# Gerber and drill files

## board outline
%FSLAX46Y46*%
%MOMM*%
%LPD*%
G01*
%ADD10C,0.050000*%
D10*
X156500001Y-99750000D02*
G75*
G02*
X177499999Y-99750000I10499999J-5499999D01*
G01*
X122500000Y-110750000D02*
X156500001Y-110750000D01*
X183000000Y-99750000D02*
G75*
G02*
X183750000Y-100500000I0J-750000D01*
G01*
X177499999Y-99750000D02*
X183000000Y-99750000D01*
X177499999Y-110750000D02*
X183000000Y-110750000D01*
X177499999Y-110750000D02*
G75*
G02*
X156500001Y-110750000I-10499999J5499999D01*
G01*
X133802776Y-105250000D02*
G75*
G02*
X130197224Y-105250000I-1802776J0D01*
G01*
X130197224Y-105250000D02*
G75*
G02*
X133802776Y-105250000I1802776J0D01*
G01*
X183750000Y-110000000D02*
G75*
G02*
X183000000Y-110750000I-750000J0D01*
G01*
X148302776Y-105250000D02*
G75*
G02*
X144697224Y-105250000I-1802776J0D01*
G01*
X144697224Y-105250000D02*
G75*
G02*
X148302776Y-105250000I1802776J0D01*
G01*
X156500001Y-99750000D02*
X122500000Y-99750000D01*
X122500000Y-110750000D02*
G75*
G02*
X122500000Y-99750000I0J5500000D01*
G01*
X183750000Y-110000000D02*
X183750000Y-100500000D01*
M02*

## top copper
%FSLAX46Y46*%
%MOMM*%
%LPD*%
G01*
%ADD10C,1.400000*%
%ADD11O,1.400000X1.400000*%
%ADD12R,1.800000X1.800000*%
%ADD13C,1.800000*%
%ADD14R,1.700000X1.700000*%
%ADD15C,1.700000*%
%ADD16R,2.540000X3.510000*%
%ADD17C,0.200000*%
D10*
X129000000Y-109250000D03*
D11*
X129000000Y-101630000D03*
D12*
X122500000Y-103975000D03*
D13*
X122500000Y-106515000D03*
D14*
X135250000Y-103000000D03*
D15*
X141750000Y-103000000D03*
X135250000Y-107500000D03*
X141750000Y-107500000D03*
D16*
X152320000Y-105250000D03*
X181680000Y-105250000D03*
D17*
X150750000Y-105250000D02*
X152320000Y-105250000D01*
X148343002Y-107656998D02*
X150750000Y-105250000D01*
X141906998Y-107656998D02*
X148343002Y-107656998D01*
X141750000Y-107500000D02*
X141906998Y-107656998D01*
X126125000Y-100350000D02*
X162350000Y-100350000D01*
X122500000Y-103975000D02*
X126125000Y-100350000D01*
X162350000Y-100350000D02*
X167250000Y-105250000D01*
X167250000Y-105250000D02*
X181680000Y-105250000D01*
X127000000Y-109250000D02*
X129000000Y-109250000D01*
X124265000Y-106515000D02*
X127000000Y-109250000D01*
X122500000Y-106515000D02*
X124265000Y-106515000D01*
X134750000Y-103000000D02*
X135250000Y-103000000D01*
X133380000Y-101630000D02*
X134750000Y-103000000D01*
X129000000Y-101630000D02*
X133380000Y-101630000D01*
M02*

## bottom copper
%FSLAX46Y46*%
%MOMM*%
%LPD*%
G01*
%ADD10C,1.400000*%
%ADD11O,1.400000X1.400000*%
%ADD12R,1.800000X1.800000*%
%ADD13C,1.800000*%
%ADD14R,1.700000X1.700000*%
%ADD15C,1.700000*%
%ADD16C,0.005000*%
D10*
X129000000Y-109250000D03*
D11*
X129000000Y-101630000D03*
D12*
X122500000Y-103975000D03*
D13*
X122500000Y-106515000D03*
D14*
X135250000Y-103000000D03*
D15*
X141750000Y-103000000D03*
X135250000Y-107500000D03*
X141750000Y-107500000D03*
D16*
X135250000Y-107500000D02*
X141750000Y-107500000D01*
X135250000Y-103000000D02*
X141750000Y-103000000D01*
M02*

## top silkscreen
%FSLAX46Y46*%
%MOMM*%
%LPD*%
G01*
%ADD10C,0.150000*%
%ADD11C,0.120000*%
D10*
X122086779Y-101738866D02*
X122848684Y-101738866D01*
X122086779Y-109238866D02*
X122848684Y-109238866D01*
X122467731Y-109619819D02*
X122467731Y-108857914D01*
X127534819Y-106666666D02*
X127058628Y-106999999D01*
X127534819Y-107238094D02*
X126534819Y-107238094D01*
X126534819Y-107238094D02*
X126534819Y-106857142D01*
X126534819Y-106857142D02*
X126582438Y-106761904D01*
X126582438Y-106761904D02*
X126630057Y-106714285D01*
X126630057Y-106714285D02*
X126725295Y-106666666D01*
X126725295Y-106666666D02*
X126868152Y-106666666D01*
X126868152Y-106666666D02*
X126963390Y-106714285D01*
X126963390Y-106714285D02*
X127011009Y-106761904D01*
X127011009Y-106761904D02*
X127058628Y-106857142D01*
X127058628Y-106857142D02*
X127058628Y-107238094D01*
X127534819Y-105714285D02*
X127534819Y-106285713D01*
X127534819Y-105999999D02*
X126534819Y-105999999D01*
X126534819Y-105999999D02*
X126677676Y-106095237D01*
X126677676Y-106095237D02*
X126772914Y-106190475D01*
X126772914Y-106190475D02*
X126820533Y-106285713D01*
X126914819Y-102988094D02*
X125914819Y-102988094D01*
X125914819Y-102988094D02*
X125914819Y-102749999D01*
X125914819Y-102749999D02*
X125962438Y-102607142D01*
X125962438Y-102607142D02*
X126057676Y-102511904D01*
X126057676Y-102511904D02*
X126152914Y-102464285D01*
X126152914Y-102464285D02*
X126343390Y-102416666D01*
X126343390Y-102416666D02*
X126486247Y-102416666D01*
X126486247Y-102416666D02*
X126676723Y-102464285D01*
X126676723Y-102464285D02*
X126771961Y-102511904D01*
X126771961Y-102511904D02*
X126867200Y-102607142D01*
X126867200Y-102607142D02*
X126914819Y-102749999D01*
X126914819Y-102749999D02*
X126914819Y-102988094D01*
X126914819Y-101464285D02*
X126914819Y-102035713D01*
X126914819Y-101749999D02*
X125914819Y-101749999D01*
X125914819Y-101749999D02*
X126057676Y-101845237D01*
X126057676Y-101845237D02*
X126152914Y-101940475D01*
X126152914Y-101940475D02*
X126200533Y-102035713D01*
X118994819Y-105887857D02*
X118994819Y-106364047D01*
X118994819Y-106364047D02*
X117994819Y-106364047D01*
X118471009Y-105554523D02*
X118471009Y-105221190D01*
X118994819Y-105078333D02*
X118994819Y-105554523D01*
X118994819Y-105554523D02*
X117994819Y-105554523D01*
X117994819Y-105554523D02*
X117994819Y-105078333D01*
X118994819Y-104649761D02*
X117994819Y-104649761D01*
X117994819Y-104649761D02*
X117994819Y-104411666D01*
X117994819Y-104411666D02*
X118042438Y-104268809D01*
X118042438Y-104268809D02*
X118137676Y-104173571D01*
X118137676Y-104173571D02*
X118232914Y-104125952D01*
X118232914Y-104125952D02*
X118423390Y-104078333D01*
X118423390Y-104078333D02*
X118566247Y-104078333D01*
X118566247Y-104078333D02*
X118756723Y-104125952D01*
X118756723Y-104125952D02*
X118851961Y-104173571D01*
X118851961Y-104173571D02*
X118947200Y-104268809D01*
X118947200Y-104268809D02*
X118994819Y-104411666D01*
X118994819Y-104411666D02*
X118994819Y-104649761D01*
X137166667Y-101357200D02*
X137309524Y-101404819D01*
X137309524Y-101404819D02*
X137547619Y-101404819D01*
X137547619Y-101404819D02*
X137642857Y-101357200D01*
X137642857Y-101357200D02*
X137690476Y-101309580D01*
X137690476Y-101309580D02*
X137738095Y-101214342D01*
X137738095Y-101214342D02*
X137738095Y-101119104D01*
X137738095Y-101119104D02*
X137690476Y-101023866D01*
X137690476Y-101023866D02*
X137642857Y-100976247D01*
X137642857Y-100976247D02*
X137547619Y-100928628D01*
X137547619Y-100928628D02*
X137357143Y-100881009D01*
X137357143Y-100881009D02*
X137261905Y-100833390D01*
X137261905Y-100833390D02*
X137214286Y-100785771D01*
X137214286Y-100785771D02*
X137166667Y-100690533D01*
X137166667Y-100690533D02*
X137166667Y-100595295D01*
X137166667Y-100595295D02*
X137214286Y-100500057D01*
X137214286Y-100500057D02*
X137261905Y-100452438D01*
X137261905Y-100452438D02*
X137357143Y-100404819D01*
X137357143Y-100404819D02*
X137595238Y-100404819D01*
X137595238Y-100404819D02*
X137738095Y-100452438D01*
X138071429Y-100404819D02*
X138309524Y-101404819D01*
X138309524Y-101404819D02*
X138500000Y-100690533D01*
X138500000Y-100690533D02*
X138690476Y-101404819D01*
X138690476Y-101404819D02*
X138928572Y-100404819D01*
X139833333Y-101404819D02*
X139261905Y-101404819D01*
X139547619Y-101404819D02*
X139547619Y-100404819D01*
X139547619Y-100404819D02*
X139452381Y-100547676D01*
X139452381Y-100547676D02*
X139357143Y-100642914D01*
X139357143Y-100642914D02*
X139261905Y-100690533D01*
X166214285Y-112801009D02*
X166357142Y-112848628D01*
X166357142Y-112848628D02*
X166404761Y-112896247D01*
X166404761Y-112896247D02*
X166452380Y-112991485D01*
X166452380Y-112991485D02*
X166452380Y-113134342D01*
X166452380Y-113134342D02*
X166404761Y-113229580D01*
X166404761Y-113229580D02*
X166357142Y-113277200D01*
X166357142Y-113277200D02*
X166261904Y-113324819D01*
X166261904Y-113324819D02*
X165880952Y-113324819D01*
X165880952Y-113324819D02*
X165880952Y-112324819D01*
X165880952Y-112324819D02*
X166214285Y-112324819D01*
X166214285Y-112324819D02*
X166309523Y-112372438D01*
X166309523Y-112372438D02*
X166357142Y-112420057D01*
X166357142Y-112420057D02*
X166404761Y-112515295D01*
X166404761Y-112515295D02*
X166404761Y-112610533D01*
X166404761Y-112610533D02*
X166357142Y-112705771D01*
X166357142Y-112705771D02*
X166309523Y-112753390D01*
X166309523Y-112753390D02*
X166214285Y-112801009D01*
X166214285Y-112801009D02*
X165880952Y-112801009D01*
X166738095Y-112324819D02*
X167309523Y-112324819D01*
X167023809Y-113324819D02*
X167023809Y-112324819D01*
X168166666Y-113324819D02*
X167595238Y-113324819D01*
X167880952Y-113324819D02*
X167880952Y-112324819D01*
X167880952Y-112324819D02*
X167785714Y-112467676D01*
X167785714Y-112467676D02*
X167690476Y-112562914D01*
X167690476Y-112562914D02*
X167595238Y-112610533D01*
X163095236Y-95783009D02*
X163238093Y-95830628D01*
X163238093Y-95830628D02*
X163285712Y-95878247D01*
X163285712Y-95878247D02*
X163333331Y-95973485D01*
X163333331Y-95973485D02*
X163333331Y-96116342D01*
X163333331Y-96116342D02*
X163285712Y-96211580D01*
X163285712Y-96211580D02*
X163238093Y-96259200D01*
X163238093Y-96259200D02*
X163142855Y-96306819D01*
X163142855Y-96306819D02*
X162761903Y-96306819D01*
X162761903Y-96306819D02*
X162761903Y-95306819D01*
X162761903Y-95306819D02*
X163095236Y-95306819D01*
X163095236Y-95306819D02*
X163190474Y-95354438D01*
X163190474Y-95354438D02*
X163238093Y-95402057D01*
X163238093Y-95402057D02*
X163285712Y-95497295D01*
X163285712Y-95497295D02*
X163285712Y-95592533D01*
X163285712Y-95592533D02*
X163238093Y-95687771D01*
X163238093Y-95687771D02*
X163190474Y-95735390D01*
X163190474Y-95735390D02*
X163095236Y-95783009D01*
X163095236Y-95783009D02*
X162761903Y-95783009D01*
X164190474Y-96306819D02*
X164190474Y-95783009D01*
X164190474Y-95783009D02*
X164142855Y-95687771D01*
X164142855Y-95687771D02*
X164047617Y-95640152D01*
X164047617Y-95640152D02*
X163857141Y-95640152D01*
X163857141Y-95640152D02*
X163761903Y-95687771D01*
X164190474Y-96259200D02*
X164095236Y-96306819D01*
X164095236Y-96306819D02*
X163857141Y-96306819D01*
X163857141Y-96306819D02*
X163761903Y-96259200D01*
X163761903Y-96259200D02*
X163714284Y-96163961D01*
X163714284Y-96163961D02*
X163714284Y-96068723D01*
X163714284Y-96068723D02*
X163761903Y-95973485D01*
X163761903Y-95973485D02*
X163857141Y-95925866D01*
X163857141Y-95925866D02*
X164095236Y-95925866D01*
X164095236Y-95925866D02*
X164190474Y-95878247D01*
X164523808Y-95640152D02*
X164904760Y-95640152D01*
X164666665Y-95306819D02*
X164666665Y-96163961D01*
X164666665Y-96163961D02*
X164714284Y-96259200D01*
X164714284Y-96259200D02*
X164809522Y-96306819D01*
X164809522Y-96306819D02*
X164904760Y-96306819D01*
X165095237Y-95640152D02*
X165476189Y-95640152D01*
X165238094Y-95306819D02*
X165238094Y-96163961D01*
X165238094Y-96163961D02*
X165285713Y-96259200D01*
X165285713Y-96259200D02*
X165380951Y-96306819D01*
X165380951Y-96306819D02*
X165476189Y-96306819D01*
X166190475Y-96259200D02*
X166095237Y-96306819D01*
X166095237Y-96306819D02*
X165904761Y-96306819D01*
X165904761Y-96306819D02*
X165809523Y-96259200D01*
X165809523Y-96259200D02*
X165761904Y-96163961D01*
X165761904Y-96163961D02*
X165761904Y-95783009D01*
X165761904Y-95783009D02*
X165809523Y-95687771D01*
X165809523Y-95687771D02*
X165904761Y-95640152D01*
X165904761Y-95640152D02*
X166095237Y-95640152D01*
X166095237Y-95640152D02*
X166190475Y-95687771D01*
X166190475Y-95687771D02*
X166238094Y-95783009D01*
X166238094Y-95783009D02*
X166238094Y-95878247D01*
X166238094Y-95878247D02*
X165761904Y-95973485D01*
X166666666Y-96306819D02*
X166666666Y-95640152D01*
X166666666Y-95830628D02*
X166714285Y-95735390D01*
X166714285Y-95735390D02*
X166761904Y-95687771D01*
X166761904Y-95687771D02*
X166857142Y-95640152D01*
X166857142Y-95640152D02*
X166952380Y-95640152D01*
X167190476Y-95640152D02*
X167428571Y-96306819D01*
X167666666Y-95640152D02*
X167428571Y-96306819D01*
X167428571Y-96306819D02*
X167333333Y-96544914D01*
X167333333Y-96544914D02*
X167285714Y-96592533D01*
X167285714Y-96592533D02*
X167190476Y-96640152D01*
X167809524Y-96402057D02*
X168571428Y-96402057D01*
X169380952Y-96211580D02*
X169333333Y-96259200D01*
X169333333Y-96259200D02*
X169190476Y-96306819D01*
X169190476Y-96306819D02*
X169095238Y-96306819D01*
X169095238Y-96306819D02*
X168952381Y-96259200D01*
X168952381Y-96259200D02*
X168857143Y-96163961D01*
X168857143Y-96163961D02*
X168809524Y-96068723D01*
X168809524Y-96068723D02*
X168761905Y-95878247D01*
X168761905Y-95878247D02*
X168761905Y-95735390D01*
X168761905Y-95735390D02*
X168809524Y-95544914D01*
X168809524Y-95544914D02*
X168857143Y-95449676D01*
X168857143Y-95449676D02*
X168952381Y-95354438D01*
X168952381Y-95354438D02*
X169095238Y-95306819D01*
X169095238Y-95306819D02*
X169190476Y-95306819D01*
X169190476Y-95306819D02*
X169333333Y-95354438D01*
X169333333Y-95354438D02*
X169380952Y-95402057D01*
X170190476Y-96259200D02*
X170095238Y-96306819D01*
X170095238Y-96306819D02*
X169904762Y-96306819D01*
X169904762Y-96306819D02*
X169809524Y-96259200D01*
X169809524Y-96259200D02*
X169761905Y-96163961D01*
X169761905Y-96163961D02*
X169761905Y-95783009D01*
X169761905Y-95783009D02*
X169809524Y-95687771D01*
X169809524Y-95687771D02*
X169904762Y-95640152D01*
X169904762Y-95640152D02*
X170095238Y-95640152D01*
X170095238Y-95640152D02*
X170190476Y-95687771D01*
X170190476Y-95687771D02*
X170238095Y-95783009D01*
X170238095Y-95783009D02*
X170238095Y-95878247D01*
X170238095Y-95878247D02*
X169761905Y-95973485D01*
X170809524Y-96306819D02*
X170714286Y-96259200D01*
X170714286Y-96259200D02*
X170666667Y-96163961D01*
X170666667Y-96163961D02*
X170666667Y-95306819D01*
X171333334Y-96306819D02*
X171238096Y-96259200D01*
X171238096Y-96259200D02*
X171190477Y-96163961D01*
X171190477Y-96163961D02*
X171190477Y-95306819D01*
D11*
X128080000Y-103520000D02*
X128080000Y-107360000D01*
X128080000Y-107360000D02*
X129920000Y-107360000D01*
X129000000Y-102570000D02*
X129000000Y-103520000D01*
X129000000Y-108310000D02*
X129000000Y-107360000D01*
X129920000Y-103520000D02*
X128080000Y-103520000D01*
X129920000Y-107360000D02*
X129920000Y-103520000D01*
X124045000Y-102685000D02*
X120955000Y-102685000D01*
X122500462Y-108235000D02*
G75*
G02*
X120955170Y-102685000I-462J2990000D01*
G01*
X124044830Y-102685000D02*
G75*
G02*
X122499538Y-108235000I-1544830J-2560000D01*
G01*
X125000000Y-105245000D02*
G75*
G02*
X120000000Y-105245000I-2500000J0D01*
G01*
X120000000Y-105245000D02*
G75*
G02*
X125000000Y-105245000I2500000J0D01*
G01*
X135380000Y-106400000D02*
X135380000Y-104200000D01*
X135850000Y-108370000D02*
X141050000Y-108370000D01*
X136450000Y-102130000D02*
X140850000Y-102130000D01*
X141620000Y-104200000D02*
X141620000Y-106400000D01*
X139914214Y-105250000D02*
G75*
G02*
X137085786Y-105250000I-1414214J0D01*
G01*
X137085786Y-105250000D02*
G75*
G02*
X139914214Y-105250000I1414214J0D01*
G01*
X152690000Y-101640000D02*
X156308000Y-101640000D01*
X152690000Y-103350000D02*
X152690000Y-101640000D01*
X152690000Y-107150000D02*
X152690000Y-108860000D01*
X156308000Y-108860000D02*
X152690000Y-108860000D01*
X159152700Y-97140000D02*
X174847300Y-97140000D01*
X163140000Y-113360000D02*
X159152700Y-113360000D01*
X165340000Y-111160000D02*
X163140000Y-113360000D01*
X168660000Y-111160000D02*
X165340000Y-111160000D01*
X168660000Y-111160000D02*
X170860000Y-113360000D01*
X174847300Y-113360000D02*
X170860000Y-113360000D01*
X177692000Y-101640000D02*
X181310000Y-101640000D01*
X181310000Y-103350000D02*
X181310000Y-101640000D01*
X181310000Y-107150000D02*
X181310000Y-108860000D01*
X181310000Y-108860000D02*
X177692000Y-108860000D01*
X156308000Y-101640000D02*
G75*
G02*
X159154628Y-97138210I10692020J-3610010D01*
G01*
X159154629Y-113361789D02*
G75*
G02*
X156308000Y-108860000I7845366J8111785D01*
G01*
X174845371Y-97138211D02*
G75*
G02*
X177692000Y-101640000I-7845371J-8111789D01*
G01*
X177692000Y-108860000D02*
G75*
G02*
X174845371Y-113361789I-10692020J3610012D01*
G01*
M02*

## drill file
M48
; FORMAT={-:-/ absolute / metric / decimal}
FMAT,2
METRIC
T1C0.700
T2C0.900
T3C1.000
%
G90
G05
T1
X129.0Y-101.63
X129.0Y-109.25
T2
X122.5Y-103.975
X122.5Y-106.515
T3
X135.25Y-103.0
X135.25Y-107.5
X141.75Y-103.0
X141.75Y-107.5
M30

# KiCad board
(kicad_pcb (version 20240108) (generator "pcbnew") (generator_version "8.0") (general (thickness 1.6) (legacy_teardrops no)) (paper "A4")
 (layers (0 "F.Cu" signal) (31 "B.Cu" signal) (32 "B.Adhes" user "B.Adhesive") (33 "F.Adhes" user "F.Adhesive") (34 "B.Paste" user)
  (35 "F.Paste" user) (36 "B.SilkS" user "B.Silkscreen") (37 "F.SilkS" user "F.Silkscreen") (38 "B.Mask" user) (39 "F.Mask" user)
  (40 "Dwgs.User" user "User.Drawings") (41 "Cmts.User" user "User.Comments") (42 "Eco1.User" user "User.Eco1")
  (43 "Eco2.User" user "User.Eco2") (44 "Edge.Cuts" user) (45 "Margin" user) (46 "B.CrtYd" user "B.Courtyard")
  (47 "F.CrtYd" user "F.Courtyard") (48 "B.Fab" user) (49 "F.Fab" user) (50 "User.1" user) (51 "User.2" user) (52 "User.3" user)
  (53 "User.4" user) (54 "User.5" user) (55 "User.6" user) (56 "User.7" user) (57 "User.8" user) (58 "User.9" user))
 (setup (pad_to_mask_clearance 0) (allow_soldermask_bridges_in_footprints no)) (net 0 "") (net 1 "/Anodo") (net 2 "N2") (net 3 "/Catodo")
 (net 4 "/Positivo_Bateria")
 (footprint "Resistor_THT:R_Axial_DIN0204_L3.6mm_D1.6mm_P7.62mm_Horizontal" (layer "F.Cu") (at 129 109.25 90)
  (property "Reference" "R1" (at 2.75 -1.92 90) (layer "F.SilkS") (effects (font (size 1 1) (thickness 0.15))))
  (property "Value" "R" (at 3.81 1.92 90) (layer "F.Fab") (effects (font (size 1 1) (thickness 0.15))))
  (fp_line (start 5.73 -0.92) (end 1.89 -0.92) (stroke (width 0.12) (type solid)) (layer "F.SilkS"))
  (fp_line (start 1.89 -0.92) (end 1.89 0.92) (stroke (width 0.12) (type solid)) (layer "F.SilkS"))
  (fp_line (start 6.68 0) (end 5.73 0) (stroke (width 0.12) (type solid)) (layer "F.SilkS"))
  (fp_line (start 0.94 0) (end 1.89 0) (stroke (width 0.12) (type solid)) (layer "F.SilkS"))
  (fp_line (start 5.73 0.92) (end 5.73 -0.92) (stroke (width 0.12) (type solid)) (layer "F.SilkS"))
  (fp_line (start 1.89 0.92) (end 5.73 0.92) (stroke (width 0.12) (type solid)) (layer "F.SilkS"))
  (pad "1" thru_hole circle (at 0 0 90) (size 1.4 1.4) (drill 0.7) (layers "*.Cu" "*.Mask") (remove_unused_layers no) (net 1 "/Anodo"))
  (pad "2" thru_hole oval (at 7.62 0 90) (size 1.4 1.4) (drill 0.7) (layers "*.Cu" "*.Mask") (remove_unused_layers no) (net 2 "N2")))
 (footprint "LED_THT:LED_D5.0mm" (layer "F.Cu") (at 122.5 103.975 -90)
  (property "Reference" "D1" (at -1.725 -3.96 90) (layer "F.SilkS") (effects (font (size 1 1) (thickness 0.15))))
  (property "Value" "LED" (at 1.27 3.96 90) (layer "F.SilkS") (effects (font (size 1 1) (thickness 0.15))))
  (fp_line (start -1.29 -1.545) (end -1.29 1.545) (stroke (width 0.12) (type solid)) (layer "F.SilkS"))
  (fp_arc (start 4.26 -0.000462) (mid 2.072002 2.880433) (end -1.29 1.54483) (stroke (width 0.12) (type solid)) (layer "F.SilkS"))
  (fp_arc (start -1.29 -1.54483) (mid 2.072002 -2.880433) (end 4.26 0.000462) (stroke (width 0.12) (type solid)) (layer "F.SilkS"))
  (fp_circle (center 1.27 0) (end 3.77 0) (stroke (width 0.12) (type solid)) (fill none) (layer "F.SilkS"))
  (pad "1" thru_hole rect (at 0 0 270) (size 1.8 1.8) (drill 0.9) (layers "*.Cu" "*.Mask") (remove_unused_layers no) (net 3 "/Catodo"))
  (pad "2" thru_hole circle (at 2.54 0 270) (size 1.8 1.8) (drill 0.9) (layers "*.Cu" "*.Mask") (remove_unused_layers no) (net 1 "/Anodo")))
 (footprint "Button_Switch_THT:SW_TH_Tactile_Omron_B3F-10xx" (layer "F.Cu") (at 135.25 103)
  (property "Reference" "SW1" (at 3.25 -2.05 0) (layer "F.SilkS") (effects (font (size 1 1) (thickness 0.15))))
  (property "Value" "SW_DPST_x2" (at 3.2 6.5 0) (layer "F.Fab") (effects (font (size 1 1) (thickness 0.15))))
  (fp_line (start 0.13 3.4) (end 0.13 1.2) (stroke (width 0.12) (type solid)) (layer "F.SilkS"))
  (fp_line (start 0.6 5.37) (end 5.8 5.37) (stroke (width 0.12) (type solid)) (layer "F.SilkS"))
  (fp_line (start 1.2 -0.87) (end 5.6 -0.87) (stroke (width 0.12) (type solid)) (layer "F.SilkS"))
  (fp_line (start 6.37 1.2) (end 6.37 3.4) (stroke (width 0.12) (type solid)) (layer "F.SilkS"))
  (fp_circle (center 3.25 2.25) (end 4.25 3.25) (stroke (width 0.12) (type solid)) (fill none) (layer "F.SilkS"))
  (pad "1" thru_hole rect (at 0 0) (size 1.7 1.7) (drill 1) (layers "*.Cu" "*.Mask") (remove_unused_layers no) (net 2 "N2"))
  (pad "1" thru_hole circle (at 6.5 0) (size 1.7 1.7) (drill 1) (layers "*.Cu" "*.Mask") (remove_unused_layers no) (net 2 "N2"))
  (pad "2" thru_hole circle (at 0 4.5) (size 1.7 1.7) (drill 1) (layers "*.Cu" "*.Mask") (remove_unused_layers no)
   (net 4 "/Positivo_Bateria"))
  (pad "2" thru_hole circle (at 6.5 4.5) (size 1.7 1.7) (drill 1) (layers "*.Cu" "*.Mask") (remove_unused_layers no)
   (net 4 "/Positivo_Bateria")))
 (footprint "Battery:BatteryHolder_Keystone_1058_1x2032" (layer "F.Cu") (at 167 105.25)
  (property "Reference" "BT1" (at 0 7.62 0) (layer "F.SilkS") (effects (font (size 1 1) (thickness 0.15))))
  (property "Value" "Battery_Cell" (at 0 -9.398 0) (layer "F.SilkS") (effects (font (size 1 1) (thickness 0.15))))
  (fp_line (start -14.31 -3.61) (end -10.692 -3.61) (stroke (width 0.12) (type solid)) (layer "F.SilkS"))
  (fp_line (start -14.31 -1.9) (end -14.31 -3.61) (stroke (width 0.12) (type solid)) (layer "F.SilkS"))
  (fp_line (start -14.31 1.9) (end -14.31 3.61) (stroke (width 0.12) (type solid)) (layer "F.SilkS"))
  (fp_line (start -10.692 3.61) (end -14.31 3.61) (stroke (width 0.12) (type solid)) (layer "F.SilkS"))
  (fp_line (start -7.8473 -8.11) (end 7.8473 -8.11) (stroke (width 0.12) (type solid)) (layer "F.SilkS"))
  (fp_line (start -3.86 8.11) (end -7.8473 8.11) (stroke (width 0.12) (type solid)) (layer "F.SilkS"))
  (fp_line (start -1.66 5.91) (end -3.86 8.11) (stroke (width 0.12) (type solid)) (layer "F.SilkS"))
  (fp_line (start 1.66 5.91) (end -1.66 5.91) (stroke (width 0.12) (type solid)) (layer "F.SilkS"))
  (fp_line (start 1.66 5.91) (end 3.86 8.11) (stroke (width 0.12) (type solid)) (layer "F.SilkS"))
  (fp_line (start 7.8473 8.11) (end 3.86 8.11) (stroke (width 0.12) (type solid)) (layer "F.SilkS"))
  (fp_line (start 10.692 -3.61) (end 14.31 -3.61) (stroke (width 0.12) (type solid)) (layer "F.SilkS"))
  (fp_line (start 14.31 -1.9) (end 14.31 -3.61) (stroke (width 0.12) (type solid)) (layer "F.SilkS"))
  (fp_line (start 14.31 1.9) (end 14.31 3.61) (stroke (width 0.12) (type solid)) (layer "F.SilkS"))
  (fp_line (start 14.31 3.61) (end 10.692 3.61) (stroke (width 0.12) (type solid)) (layer "F.SilkS"))
  (fp_arc (start -10.692 -3.61) (mid -9.538084 -6.031244) (end -7.845371 -8.111789) (stroke (width 0.12) (type solid)) (layer "F.SilkS"))
  (fp_arc (start -7.845371 8.111789) (mid -9.538085 6.031244) (end -10.692 3.61) (stroke (width 0.12) (type solid)) (layer "F.SilkS"))
  (fp_arc (start 7.845371 -8.111789) (mid 9.538085 -6.031244) (end 10.692 -3.61) (stroke (width 0.12) (type solid)) (layer "F.SilkS"))
  (fp_arc (start 10.692 3.61) (mid 9.538084 6.031244) (end 7.845371 8.111789) (stroke (width 0.12) (type solid)) (layer "F.SilkS"))
  (pad "1" smd rect (at -14.68 0) (size 2.54 3.51) (layers "F.Cu" "F.Paste" "F.Mask") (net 4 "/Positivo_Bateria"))
  (pad "2" smd rect (at 14.68 0) (size 2.54 3.51) (layers "F.Cu" "F.Paste" "F.Mask") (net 3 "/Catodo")))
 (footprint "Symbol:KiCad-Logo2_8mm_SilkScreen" (layer "B.Cu") (at 167.25 104.75 180)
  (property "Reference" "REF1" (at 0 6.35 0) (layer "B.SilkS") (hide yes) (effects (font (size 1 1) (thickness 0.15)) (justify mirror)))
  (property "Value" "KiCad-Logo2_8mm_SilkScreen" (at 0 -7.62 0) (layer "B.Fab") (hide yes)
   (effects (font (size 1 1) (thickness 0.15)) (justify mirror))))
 (gr_arc (start 156.500001 99.75) (mid 167 93.396731) (end 177.499999 99.75) (stroke (width 0.05) (type default)) (layer "Edge.Cuts"))
 (gr_line (start 122.5 110.75) (end 156.500001 110.75) (stroke (width 0.05) (type default)) (layer "Edge.Cuts"))
 (gr_arc (start 183 99.75) (mid 183.53033 99.96967) (end 183.75 100.5) (stroke (width 0.05) (type default)) (layer "Edge.Cuts"))
 (gr_line (start 177.499999 99.75) (end 183 99.75) (stroke (width 0.05) (type default)) (layer "Edge.Cuts"))
 (gr_line (start 177.499999 110.75) (end 183 110.75) (stroke (width 0.05) (type default)) (layer "Edge.Cuts"))
 (gr_arc (start 177.499999 110.75) (mid 167 117.103269) (end 156.500001 110.75) (stroke (width 0.05) (type default)) (layer "Edge.Cuts"))
 (gr_circle (center 132 105.25) (end 133 106.75) (stroke (width 0.05) (type default)) (fill none) (layer "Edge.Cuts"))
 (gr_arc (start 183.75 110) (mid 183.53033 110.53033) (end 183 110.75) (stroke (width 0.05) (type default)) (layer "Edge.Cuts"))
 (gr_circle (center 146.5 105.25) (end 147.5 106.75) (stroke (width 0.05) (type default)) (fill none) (layer "Edge.Cuts"))
 (gr_line (start 156.500001 99.75) (end 122.5 99.75) (stroke (width 0.05) (type default)) (layer "Edge.Cuts"))
 (gr_arc (start 122.5 110.75) (mid 117 105.25) (end 122.5 99.75) (stroke (width 0.05) (type default)) (layer "Edge.Cuts"))
 (gr_line (start 183.75 110) (end 183.75 100.5) (stroke (width 0.05) (type default)) (layer "Edge.Cuts"))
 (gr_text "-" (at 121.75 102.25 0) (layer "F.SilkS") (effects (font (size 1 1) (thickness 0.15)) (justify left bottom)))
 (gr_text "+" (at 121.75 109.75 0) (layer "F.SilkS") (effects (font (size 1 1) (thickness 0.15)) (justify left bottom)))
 (segment (start 150.75 105.25) (end 152.32 105.25) (width 0.2) (layer "F.Cu") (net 4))
 (segment (start 148.343002 107.656998) (end 150.75 105.25) (width 0.2) (layer "F.Cu") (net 4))
 (segment (start 141.906998 107.656998) (end 148.343002 107.656998) (width 0.2) (layer "F.Cu") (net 4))
 (segment (start 141.75 107.5) (end 141.906998 107.656998) (width 0.2) (layer "F.Cu") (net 4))
 (segment (start 135.25 107.5) (end 141.75 107.5) (width 0.005) (layer "B.Cu") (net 4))
 (segment (start 126.125 100.35) (end 162.35 100.35) (width 0.2) (layer "F.Cu") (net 3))
 (segment (start 122.5 103.975) (end 126.125 100.35) (width 0.2) (layer "F.Cu") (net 3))
 (segment (start 162.35 100.35) (end 167.25 105.25) (width 0.2) (layer "F.Cu") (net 3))
 (segment (start 167.25 105.25) (end 181.68 105.25) (width 0.2) (layer "F.Cu") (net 3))
 (segment (start 127 109.25) (end 129 109.25) (width 0.2) (layer "F.Cu") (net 1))
 (segment (start 124.265 106.515) (end 127 109.25) (width 0.2) (layer "F.Cu") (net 1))
 (segment (start 122.5 106.515) (end 124.265 106.515) (width 0.2) (layer "F.Cu") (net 1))
 (segment (start 134.75 103) (end 135.25 103) (width 0.2) (layer "F.Cu") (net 2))
 (segment (start 133.38 101.63) (end 134.75 103) (width 0.2) (layer "F.Cu") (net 2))
 (segment (start 129 101.63) (end 133.38 101.63) (width 0.2) (layer "F.Cu") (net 2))
 (segment (start 135.25 103) (end 141.75 103) (width 0.005) (layer "B.Cu") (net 2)))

